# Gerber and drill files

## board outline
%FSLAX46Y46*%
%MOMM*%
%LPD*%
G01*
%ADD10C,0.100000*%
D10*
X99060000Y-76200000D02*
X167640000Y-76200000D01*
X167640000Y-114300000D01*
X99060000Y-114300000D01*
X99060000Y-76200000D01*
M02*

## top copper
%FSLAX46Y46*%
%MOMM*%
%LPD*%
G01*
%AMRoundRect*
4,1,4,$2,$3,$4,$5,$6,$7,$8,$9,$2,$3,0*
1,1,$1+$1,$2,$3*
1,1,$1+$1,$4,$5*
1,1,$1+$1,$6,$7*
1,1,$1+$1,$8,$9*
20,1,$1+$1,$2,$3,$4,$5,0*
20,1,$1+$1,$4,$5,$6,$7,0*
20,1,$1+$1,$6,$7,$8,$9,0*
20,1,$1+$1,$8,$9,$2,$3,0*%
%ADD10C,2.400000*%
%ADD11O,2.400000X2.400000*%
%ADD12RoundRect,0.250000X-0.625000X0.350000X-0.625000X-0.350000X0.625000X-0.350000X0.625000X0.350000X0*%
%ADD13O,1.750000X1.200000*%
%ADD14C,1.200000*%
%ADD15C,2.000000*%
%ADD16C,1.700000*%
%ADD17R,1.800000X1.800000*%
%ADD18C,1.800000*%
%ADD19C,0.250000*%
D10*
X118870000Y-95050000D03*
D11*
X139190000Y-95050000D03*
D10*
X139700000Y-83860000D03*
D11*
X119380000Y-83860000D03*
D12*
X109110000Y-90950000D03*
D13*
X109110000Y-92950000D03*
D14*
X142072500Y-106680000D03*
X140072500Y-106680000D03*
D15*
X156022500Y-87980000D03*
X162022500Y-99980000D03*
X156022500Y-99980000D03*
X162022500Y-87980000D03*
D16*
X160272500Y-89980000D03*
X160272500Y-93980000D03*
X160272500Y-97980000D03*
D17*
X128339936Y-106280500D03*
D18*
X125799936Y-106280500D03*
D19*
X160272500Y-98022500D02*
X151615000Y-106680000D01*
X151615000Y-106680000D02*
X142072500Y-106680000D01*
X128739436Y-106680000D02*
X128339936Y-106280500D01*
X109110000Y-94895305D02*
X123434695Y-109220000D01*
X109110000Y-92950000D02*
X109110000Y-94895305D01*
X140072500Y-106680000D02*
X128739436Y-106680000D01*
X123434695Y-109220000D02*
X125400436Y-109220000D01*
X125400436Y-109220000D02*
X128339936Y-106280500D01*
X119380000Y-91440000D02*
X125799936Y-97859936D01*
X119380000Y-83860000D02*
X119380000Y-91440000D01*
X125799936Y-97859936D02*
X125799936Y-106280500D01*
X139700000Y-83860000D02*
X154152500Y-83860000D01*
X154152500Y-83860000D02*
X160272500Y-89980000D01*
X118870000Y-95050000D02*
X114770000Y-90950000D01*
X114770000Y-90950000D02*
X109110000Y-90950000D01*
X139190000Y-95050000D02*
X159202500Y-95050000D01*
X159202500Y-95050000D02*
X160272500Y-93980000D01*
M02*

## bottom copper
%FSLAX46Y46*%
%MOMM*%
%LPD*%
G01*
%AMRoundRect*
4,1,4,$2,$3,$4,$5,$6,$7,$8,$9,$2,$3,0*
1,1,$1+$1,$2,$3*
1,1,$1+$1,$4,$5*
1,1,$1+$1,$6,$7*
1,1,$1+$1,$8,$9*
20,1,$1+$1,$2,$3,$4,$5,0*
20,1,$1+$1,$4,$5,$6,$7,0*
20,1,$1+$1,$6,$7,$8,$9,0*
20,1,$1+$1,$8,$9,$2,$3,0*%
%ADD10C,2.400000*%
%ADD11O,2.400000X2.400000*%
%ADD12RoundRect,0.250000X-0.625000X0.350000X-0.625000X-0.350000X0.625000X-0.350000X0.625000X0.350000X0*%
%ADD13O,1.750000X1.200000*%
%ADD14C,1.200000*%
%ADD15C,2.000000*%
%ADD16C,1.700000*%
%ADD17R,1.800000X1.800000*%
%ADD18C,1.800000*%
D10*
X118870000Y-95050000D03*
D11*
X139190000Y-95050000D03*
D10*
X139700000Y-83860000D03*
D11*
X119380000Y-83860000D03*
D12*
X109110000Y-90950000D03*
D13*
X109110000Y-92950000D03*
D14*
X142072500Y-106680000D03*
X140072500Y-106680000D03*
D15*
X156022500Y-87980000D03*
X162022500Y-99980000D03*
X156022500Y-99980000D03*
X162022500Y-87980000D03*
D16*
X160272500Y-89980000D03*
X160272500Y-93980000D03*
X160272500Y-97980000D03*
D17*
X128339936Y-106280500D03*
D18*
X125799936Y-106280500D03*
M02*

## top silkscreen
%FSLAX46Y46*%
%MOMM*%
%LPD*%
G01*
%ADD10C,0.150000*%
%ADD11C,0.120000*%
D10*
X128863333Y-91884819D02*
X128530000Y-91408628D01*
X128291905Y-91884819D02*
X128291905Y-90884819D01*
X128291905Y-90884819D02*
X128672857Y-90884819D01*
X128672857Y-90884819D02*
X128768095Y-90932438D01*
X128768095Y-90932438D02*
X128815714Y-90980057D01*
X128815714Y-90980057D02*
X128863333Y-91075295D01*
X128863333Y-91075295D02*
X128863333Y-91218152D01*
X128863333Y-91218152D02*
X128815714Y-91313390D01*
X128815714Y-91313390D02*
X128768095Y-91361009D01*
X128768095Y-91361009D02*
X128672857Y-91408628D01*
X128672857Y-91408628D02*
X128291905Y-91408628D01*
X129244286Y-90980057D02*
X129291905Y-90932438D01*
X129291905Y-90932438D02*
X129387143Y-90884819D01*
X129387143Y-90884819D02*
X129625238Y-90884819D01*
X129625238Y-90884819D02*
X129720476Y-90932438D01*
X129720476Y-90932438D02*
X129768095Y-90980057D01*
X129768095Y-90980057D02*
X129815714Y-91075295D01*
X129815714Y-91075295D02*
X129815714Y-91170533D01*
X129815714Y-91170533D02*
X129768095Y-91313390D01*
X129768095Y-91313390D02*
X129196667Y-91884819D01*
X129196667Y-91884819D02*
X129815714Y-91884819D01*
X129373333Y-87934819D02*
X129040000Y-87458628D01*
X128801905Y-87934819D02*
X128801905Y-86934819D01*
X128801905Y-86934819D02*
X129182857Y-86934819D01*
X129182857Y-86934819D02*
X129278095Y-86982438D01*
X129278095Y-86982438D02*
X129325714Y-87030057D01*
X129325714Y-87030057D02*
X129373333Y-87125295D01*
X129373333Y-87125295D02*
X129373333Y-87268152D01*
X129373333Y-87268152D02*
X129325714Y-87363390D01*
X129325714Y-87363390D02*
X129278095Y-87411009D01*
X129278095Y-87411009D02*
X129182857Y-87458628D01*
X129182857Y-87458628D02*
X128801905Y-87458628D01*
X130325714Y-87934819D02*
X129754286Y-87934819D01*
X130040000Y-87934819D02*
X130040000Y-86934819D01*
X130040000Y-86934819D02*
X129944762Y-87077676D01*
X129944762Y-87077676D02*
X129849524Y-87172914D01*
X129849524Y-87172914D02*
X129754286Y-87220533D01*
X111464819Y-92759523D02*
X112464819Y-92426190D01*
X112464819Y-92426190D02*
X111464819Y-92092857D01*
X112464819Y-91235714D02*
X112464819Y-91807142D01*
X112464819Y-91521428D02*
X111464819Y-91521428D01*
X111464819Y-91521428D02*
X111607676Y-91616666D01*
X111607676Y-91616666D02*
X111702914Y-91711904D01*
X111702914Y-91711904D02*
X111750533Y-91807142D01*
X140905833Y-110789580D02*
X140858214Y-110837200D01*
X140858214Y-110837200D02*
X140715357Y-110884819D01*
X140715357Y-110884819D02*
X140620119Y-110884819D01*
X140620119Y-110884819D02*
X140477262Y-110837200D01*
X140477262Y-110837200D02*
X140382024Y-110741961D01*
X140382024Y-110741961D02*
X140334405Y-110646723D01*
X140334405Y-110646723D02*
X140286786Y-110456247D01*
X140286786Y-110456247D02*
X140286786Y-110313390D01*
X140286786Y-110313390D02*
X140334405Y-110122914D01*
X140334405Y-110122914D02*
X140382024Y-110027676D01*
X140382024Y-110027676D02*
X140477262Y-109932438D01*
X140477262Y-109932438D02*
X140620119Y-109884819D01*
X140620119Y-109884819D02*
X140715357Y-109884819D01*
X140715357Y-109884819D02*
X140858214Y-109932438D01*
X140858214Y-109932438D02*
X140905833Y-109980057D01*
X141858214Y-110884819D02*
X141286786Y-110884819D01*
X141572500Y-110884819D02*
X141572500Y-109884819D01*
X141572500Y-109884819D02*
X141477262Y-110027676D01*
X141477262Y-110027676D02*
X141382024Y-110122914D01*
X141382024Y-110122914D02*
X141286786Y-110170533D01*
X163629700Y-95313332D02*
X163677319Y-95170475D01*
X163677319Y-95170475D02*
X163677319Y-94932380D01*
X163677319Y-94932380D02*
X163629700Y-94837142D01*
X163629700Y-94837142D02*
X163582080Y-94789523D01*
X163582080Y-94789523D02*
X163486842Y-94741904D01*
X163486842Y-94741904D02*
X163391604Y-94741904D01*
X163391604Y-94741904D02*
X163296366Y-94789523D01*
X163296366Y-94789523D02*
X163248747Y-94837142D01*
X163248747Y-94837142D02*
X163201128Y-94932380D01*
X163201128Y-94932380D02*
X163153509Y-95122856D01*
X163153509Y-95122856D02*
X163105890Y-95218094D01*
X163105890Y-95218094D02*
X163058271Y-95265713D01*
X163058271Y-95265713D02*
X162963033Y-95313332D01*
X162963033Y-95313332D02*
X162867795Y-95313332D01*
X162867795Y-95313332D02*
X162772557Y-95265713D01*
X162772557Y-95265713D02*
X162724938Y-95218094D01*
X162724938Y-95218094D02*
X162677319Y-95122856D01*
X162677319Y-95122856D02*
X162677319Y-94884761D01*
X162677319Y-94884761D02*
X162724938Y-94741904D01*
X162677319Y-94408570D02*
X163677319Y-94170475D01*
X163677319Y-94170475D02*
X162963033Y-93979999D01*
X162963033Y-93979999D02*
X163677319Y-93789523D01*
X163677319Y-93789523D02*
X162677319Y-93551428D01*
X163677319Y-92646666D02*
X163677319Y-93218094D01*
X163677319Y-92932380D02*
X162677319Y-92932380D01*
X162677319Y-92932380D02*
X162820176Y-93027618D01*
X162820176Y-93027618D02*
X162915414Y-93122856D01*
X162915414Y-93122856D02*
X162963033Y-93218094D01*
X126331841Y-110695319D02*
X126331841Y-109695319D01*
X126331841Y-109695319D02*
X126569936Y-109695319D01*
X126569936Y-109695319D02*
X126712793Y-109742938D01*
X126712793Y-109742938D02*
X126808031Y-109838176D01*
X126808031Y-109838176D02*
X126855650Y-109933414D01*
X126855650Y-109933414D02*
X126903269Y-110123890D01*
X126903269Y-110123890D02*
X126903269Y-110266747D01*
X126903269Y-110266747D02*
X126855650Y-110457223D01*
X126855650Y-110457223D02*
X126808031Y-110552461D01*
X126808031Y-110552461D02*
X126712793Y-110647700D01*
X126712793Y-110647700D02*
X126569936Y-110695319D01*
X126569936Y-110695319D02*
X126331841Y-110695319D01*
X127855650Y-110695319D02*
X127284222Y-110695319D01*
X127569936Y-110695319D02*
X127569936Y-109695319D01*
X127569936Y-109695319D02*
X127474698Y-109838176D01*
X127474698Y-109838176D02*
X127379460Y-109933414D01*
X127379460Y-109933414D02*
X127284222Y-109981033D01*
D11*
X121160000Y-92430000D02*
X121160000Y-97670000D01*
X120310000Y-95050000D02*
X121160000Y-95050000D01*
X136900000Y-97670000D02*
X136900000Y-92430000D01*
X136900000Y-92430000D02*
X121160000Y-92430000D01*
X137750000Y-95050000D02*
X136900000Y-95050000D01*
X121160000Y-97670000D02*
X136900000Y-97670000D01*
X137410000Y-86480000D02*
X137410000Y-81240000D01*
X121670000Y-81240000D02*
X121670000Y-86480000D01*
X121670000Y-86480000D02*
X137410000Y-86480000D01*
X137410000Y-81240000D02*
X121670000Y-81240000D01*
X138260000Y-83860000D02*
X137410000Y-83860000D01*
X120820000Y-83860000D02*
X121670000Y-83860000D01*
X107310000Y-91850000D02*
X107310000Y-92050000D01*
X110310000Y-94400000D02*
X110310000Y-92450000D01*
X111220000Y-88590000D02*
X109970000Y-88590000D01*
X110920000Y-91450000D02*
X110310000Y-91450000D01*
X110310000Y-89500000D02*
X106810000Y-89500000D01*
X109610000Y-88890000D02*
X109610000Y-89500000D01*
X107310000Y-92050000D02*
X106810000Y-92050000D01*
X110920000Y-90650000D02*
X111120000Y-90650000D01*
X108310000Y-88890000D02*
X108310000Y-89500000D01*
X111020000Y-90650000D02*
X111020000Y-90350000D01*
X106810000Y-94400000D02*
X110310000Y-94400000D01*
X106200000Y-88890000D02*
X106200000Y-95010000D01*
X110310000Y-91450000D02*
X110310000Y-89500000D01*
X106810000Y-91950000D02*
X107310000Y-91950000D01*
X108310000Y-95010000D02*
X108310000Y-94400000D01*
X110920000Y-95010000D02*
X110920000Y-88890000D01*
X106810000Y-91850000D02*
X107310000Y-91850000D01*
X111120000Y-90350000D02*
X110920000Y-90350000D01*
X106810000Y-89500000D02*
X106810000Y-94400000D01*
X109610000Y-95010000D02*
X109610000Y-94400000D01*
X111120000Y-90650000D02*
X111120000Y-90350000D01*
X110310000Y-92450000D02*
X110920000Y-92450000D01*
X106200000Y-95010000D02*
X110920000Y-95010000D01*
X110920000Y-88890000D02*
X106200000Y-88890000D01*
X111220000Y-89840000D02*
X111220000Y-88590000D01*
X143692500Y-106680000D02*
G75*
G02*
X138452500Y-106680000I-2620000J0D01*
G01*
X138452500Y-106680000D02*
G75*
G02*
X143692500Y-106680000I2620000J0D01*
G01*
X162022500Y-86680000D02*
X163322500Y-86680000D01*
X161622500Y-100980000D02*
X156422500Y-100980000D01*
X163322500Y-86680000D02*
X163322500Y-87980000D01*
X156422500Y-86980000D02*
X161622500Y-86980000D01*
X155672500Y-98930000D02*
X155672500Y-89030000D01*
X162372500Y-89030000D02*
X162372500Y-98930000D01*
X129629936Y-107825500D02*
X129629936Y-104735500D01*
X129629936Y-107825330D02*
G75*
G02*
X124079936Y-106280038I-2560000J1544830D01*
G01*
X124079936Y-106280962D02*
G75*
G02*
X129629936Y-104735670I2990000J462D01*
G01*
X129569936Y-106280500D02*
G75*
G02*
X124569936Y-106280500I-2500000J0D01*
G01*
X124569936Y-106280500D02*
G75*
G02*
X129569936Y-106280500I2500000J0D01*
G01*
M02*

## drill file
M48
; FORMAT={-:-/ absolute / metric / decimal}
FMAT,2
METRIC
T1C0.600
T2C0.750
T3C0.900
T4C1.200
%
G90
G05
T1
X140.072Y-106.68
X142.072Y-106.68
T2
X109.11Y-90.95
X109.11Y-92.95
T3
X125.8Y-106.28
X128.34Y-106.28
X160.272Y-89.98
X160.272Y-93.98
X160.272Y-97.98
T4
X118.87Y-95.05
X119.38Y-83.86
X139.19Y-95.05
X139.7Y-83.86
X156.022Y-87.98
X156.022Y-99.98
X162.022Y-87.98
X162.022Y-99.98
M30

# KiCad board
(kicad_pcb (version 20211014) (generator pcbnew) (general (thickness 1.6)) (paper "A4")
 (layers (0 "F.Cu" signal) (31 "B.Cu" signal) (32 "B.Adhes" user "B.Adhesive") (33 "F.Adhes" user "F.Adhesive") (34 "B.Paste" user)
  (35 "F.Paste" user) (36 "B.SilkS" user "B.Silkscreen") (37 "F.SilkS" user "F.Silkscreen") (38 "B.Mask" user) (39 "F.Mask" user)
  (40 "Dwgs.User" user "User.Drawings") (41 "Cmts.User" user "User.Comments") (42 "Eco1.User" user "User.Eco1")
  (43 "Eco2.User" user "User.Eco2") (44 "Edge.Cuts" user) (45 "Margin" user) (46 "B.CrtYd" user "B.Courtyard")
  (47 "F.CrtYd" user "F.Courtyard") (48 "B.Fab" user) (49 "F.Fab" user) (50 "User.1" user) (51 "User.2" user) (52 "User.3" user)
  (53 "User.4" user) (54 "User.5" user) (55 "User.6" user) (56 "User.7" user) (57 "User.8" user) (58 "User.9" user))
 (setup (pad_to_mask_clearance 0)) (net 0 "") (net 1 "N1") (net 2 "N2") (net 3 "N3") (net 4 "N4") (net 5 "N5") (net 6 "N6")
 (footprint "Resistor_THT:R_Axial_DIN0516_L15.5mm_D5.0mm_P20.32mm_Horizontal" (layer "F.Cu") (at 118.87 95.05)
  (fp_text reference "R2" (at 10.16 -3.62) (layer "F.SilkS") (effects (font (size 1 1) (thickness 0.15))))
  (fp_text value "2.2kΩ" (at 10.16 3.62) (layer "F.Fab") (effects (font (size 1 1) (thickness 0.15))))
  (fp_line (start 2.29 -2.62) (end 2.29 2.62) (layer "F.SilkS") (width 0.12))
  (fp_line (start 1.44 0) (end 2.29 0) (layer "F.SilkS") (width 0.12))
  (fp_line (start 18.03 2.62) (end 18.03 -2.62) (layer "F.SilkS") (width 0.12))
  (fp_line (start 18.03 -2.62) (end 2.29 -2.62) (layer "F.SilkS") (width 0.12))
  (fp_line (start 18.88 0) (end 18.03 0) (layer "F.SilkS") (width 0.12))
  (fp_line (start 2.29 2.62) (end 18.03 2.62) (layer "F.SilkS") (width 0.12))
  (pad "1" thru_hole circle (at 0 0) (size 2.4 2.4) (drill 1.2) (layers *.Cu *.Mask) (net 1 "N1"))
  (pad "2" thru_hole oval (at 20.32 0) (size 2.4 2.4) (drill 1.2) (layers *.Cu *.Mask) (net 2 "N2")))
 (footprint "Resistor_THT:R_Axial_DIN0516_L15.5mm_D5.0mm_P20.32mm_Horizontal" (layer "F.Cu") (at 139.7 83.86 180)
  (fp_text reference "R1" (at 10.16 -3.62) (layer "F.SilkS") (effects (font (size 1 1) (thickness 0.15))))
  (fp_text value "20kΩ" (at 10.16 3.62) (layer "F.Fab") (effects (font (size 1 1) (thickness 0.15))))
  (fp_line (start 2.29 -2.62) (end 2.29 2.62) (layer "F.SilkS") (width 0.12))
  (fp_line (start 18.03 2.62) (end 18.03 -2.62) (layer "F.SilkS") (width 0.12))
  (fp_line (start 18.03 -2.62) (end 2.29 -2.62) (layer "F.SilkS") (width 0.12))
  (fp_line (start 2.29 2.62) (end 18.03 2.62) (layer "F.SilkS") (width 0.12))
  (fp_line (start 1.44 0) (end 2.29 0) (layer "F.SilkS") (width 0.12))
  (fp_line (start 18.88 0) (end 18.03 0) (layer "F.SilkS") (width 0.12))
  (pad "1" thru_hole circle (at 0 0 180) (size 2.4 2.4) (drill 1.2) (layers *.Cu *.Mask) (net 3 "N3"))
  (pad "2" thru_hole oval (at 20.32 0 180) (size 2.4 2.4) (drill 1.2) (layers *.Cu *.Mask) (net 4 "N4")))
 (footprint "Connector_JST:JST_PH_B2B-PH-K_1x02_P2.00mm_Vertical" (layer "F.Cu") (at 109.11 90.95 -90)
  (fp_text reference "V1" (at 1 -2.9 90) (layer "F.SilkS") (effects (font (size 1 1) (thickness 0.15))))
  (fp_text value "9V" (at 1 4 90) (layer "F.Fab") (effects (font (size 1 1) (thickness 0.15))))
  (fp_line (start 0.9 1.8) (end 1.1 1.8) (layer "F.SilkS") (width 0.12))
  (fp_line (start 3.45 -1.2) (end 1.5 -1.2) (layer "F.SilkS") (width 0.12))
  (fp_line (start -2.36 -2.11) (end -2.36 -0.86) (layer "F.SilkS") (width 0.12))
  (fp_line (start 0.5 -1.81) (end 0.5 -1.2) (layer "F.SilkS") (width 0.12))
  (fp_line (start -1.45 -1.2) (end -1.45 2.3) (layer "F.SilkS") (width 0.12))
  (fp_line (start -2.06 -0.5) (end -1.45 -0.5) (layer "F.SilkS") (width 0.12))
  (fp_line (start 1.1 1.8) (end 1.1 2.3) (layer "F.SilkS") (width 0.12))
  (fp_line (start -0.3 -1.81) (end -0.3 -2.01) (layer "F.SilkS") (width 0.12))
  (fp_line (start -2.06 0.8) (end -1.45 0.8) (layer "F.SilkS") (width 0.12))
  (fp_line (start -0.3 -1.91) (end -0.6 -1.91) (layer "F.SilkS") (width 0.12))
  (fp_line (start 3.45 2.3) (end 3.45 -1.2) (layer "F.SilkS") (width 0.12))
  (fp_line (start -2.06 2.91) (end 4.06 2.91) (layer "F.SilkS") (width 0.12))
  (fp_line (start 0.5 -1.2) (end -1.45 -1.2) (layer "F.SilkS") (width 0.12))
  (fp_line (start 1 2.3) (end 1 1.8) (layer "F.SilkS") (width 0.12))
  (fp_line (start 4.06 0.8) (end 3.45 0.8) (layer "F.SilkS") (width 0.12))
  (fp_line (start 4.06 -1.81) (end -2.06 -1.81) (layer "F.SilkS") (width 0.12))
  (fp_line (start 0.9 2.3) (end 0.9 1.8) (layer "F.SilkS") (width 0.12))
  (fp_line (start -0.6 -2.01) (end -0.6 -1.81) (layer "F.SilkS") (width 0.12))
  (fp_line (start -1.45 2.3) (end 3.45 2.3) (layer "F.SilkS") (width 0.12))
  (fp_line (start 4.06 -0.5) (end 3.45 -0.5) (layer "F.SilkS") (width 0.12))
  (fp_line (start -0.3 -2.01) (end -0.6 -2.01) (layer "F.SilkS") (width 0.12))
  (fp_line (start 1.5 -1.2) (end 1.5 -1.81) (layer "F.SilkS") (width 0.12))
  (fp_line (start 4.06 2.91) (end 4.06 -1.81) (layer "F.SilkS") (width 0.12))
  (fp_line (start -2.06 -1.81) (end -2.06 2.91) (layer "F.SilkS") (width 0.12))
  (fp_line (start -1.11 -2.11) (end -2.36 -2.11) (layer "F.SilkS") (width 0.12))
  (pad "1" thru_hole roundrect (at 0 0 270) (size 1.2 1.75) (drill 0.75) (layers *.Cu *.Mask) (roundrect_rratio 0.208333) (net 1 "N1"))
  (pad "2" thru_hole oval (at 2 0 270) (size 1.2 1.75) (drill 0.75) (layers *.Cu *.Mask) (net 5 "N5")))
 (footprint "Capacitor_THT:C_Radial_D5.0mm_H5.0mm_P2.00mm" (layer "F.Cu") (at 142.0725 106.68 180)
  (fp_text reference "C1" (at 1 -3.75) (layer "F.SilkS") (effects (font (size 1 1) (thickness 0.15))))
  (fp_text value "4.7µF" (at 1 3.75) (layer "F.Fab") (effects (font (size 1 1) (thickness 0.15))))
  (fp_circle (center 1 0) (end 3.62 0) (layer "F.SilkS") (width 0.12) (fill none))
  (pad "1" thru_hole circle (at 0 0 180) (size 1.2 1.2) (drill 0.6) (layers *.Cu *.Mask) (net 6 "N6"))
  (pad "2" thru_hole circle (at 2 0 180) (size 1.2 1.2) (drill 0.6) (layers *.Cu *.Mask) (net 5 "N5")))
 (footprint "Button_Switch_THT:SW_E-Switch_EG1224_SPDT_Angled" (layer "F.Cu") (at 160.2725 89.98 -90)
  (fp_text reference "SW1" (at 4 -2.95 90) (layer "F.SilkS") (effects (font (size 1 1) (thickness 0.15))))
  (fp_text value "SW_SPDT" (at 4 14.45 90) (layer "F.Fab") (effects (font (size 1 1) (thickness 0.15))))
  (fp_line (start -3.3 -1.75) (end -3.3 -3.05) (layer "F.SilkS") (width 0.12))
  (fp_line (start 11 -1.35) (end 11 3.85) (layer "F.SilkS") (width 0.12))
  (fp_line (start -3.3 -3.05) (end -2 -3.05) (layer "F.SilkS") (width 0.12))
  (fp_line (start -3 3.85) (end -3 -1.35) (layer "F.SilkS") (width 0.12))
  (fp_line (start 8.95 4.6) (end -0.95 4.6) (layer "F.SilkS") (width 0.12))
  (fp_line (start -0.95 -2.1) (end 8.95 -2.1) (layer "F.SilkS") (width 0.12))
  (pad "" thru_hole circle (at -2 4.25 270) (size 2 2) (drill 1.2) (layers *.Cu *.Mask))
  (pad "" thru_hole circle (at 10 -1.75 270) (size 2 2) (drill 1.2) (layers *.Cu *.Mask))
  (pad "" thru_hole circle (at 10 4.25 270) (size 2 2) (drill 1.2) (layers *.Cu *.Mask))
  (pad "" thru_hole circle (at -2 -1.75 270) (size 2 2) (drill 1.2) (layers *.Cu *.Mask))
  (pad "1" thru_hole circle (at 0 0 270) (size 1.7 1.7) (drill 0.9) (layers *.Cu *.Mask) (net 3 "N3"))
  (pad "2" thru_hole circle (at 4 0 270) (size 1.7 1.7) (drill 0.9) (layers *.Cu *.Mask) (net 2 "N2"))
  (pad "3" thru_hole circle (at 8 0 270) (size 1.7 1.7) (drill 0.9) (layers *.Cu *.Mask) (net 6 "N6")))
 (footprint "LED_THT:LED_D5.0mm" (layer "F.Cu") (at 128.339936 106.2805 180)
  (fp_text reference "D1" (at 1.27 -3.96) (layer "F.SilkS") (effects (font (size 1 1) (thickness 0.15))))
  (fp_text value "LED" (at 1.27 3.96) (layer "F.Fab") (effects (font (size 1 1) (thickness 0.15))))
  (fp_line (start -1.29 -1.545) (end -1.29 1.545) (layer "F.SilkS") (width 0.12))
  (fp_arc (start -1.29 -1.54483) (mid 2.072002 -2.880433) (end 4.26 0.000462) (layer "F.SilkS") (width 0.12))
  (fp_arc (start 4.26 -0.000462) (mid 2.072002 2.880433) (end -1.29 1.54483) (layer "F.SilkS") (width 0.12))
  (fp_circle (center 1.27 0) (end 3.77 0) (layer "F.SilkS") (width 0.12) (fill none))
  (pad "1" thru_hole rect (at 0 0 180) (size 1.8 1.8) (drill 0.9) (layers *.Cu *.Mask) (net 5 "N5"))
  (pad "2" thru_hole circle (at 2.54 0 180) (size 1.8 1.8) (drill 0.9) (layers *.Cu *.Mask) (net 4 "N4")))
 (gr_rect (start 167.64 114.3) (end 99.06 76.2) (layer "Edge.Cuts") (width 0.1) (fill none))
 (segment (start 160.2725 98.0225) (end 151.615 106.68) (width 0.25) (layer "F.Cu") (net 6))
 (segment (start 151.615 106.68) (end 142.0725 106.68) (width 0.25) (layer "F.Cu") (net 6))
 (segment (start 128.739436 106.68) (end 128.339936 106.2805) (width 0.25) (layer "F.Cu") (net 5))
 (segment (start 109.11 94.895305) (end 123.434695 109.22) (width 0.25) (layer "F.Cu") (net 5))
 (segment (start 109.11 92.95) (end 109.11 94.895305) (width 0.25) (layer "F.Cu") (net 5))
 (segment (start 140.0725 106.68) (end 128.739436 106.68) (width 0.25) (layer "F.Cu") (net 5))
 (segment (start 123.434695 109.22) (end 125.400436 109.22) (width 0.25) (layer "F.Cu") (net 5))
 (segment (start 125.400436 109.22) (end 128.339936 106.2805) (width 0.25) (layer "F.Cu") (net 5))
 (segment (start 119.38 91.44) (end 125.799936 97.859936) (width 0.25) (layer "F.Cu") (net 4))
 (segment (start 119.38 83.86) (end 119.38 91.44) (width 0.25) (layer "F.Cu") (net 4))
 (segment (start 125.799936 97.859936) (end 125.799936 106.2805) (width 0.25) (layer "F.Cu") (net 4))
 (segment (start 139.7 83.86) (end 154.1525 83.86) (width 0.25) (layer "F.Cu") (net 3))
 (segment (start 154.1525 83.86) (end 160.2725 89.98) (width 0.25) (layer "F.Cu") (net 3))
 (segment (start 118.87 95.05) (end 114.77 90.95) (width 0.25) (layer "F.Cu") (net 1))
 (segment (start 114.77 90.95) (end 109.11 90.95) (width 0.25) (layer "F.Cu") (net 1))
 (segment (start 139.19 95.05) (end 159.2025 95.05) (width 0.25) (layer "F.Cu") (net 2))
 (segment (start 159.2025 95.05) (end 160.2725 93.98) (width 0.25) (layer "F.Cu") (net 2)))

